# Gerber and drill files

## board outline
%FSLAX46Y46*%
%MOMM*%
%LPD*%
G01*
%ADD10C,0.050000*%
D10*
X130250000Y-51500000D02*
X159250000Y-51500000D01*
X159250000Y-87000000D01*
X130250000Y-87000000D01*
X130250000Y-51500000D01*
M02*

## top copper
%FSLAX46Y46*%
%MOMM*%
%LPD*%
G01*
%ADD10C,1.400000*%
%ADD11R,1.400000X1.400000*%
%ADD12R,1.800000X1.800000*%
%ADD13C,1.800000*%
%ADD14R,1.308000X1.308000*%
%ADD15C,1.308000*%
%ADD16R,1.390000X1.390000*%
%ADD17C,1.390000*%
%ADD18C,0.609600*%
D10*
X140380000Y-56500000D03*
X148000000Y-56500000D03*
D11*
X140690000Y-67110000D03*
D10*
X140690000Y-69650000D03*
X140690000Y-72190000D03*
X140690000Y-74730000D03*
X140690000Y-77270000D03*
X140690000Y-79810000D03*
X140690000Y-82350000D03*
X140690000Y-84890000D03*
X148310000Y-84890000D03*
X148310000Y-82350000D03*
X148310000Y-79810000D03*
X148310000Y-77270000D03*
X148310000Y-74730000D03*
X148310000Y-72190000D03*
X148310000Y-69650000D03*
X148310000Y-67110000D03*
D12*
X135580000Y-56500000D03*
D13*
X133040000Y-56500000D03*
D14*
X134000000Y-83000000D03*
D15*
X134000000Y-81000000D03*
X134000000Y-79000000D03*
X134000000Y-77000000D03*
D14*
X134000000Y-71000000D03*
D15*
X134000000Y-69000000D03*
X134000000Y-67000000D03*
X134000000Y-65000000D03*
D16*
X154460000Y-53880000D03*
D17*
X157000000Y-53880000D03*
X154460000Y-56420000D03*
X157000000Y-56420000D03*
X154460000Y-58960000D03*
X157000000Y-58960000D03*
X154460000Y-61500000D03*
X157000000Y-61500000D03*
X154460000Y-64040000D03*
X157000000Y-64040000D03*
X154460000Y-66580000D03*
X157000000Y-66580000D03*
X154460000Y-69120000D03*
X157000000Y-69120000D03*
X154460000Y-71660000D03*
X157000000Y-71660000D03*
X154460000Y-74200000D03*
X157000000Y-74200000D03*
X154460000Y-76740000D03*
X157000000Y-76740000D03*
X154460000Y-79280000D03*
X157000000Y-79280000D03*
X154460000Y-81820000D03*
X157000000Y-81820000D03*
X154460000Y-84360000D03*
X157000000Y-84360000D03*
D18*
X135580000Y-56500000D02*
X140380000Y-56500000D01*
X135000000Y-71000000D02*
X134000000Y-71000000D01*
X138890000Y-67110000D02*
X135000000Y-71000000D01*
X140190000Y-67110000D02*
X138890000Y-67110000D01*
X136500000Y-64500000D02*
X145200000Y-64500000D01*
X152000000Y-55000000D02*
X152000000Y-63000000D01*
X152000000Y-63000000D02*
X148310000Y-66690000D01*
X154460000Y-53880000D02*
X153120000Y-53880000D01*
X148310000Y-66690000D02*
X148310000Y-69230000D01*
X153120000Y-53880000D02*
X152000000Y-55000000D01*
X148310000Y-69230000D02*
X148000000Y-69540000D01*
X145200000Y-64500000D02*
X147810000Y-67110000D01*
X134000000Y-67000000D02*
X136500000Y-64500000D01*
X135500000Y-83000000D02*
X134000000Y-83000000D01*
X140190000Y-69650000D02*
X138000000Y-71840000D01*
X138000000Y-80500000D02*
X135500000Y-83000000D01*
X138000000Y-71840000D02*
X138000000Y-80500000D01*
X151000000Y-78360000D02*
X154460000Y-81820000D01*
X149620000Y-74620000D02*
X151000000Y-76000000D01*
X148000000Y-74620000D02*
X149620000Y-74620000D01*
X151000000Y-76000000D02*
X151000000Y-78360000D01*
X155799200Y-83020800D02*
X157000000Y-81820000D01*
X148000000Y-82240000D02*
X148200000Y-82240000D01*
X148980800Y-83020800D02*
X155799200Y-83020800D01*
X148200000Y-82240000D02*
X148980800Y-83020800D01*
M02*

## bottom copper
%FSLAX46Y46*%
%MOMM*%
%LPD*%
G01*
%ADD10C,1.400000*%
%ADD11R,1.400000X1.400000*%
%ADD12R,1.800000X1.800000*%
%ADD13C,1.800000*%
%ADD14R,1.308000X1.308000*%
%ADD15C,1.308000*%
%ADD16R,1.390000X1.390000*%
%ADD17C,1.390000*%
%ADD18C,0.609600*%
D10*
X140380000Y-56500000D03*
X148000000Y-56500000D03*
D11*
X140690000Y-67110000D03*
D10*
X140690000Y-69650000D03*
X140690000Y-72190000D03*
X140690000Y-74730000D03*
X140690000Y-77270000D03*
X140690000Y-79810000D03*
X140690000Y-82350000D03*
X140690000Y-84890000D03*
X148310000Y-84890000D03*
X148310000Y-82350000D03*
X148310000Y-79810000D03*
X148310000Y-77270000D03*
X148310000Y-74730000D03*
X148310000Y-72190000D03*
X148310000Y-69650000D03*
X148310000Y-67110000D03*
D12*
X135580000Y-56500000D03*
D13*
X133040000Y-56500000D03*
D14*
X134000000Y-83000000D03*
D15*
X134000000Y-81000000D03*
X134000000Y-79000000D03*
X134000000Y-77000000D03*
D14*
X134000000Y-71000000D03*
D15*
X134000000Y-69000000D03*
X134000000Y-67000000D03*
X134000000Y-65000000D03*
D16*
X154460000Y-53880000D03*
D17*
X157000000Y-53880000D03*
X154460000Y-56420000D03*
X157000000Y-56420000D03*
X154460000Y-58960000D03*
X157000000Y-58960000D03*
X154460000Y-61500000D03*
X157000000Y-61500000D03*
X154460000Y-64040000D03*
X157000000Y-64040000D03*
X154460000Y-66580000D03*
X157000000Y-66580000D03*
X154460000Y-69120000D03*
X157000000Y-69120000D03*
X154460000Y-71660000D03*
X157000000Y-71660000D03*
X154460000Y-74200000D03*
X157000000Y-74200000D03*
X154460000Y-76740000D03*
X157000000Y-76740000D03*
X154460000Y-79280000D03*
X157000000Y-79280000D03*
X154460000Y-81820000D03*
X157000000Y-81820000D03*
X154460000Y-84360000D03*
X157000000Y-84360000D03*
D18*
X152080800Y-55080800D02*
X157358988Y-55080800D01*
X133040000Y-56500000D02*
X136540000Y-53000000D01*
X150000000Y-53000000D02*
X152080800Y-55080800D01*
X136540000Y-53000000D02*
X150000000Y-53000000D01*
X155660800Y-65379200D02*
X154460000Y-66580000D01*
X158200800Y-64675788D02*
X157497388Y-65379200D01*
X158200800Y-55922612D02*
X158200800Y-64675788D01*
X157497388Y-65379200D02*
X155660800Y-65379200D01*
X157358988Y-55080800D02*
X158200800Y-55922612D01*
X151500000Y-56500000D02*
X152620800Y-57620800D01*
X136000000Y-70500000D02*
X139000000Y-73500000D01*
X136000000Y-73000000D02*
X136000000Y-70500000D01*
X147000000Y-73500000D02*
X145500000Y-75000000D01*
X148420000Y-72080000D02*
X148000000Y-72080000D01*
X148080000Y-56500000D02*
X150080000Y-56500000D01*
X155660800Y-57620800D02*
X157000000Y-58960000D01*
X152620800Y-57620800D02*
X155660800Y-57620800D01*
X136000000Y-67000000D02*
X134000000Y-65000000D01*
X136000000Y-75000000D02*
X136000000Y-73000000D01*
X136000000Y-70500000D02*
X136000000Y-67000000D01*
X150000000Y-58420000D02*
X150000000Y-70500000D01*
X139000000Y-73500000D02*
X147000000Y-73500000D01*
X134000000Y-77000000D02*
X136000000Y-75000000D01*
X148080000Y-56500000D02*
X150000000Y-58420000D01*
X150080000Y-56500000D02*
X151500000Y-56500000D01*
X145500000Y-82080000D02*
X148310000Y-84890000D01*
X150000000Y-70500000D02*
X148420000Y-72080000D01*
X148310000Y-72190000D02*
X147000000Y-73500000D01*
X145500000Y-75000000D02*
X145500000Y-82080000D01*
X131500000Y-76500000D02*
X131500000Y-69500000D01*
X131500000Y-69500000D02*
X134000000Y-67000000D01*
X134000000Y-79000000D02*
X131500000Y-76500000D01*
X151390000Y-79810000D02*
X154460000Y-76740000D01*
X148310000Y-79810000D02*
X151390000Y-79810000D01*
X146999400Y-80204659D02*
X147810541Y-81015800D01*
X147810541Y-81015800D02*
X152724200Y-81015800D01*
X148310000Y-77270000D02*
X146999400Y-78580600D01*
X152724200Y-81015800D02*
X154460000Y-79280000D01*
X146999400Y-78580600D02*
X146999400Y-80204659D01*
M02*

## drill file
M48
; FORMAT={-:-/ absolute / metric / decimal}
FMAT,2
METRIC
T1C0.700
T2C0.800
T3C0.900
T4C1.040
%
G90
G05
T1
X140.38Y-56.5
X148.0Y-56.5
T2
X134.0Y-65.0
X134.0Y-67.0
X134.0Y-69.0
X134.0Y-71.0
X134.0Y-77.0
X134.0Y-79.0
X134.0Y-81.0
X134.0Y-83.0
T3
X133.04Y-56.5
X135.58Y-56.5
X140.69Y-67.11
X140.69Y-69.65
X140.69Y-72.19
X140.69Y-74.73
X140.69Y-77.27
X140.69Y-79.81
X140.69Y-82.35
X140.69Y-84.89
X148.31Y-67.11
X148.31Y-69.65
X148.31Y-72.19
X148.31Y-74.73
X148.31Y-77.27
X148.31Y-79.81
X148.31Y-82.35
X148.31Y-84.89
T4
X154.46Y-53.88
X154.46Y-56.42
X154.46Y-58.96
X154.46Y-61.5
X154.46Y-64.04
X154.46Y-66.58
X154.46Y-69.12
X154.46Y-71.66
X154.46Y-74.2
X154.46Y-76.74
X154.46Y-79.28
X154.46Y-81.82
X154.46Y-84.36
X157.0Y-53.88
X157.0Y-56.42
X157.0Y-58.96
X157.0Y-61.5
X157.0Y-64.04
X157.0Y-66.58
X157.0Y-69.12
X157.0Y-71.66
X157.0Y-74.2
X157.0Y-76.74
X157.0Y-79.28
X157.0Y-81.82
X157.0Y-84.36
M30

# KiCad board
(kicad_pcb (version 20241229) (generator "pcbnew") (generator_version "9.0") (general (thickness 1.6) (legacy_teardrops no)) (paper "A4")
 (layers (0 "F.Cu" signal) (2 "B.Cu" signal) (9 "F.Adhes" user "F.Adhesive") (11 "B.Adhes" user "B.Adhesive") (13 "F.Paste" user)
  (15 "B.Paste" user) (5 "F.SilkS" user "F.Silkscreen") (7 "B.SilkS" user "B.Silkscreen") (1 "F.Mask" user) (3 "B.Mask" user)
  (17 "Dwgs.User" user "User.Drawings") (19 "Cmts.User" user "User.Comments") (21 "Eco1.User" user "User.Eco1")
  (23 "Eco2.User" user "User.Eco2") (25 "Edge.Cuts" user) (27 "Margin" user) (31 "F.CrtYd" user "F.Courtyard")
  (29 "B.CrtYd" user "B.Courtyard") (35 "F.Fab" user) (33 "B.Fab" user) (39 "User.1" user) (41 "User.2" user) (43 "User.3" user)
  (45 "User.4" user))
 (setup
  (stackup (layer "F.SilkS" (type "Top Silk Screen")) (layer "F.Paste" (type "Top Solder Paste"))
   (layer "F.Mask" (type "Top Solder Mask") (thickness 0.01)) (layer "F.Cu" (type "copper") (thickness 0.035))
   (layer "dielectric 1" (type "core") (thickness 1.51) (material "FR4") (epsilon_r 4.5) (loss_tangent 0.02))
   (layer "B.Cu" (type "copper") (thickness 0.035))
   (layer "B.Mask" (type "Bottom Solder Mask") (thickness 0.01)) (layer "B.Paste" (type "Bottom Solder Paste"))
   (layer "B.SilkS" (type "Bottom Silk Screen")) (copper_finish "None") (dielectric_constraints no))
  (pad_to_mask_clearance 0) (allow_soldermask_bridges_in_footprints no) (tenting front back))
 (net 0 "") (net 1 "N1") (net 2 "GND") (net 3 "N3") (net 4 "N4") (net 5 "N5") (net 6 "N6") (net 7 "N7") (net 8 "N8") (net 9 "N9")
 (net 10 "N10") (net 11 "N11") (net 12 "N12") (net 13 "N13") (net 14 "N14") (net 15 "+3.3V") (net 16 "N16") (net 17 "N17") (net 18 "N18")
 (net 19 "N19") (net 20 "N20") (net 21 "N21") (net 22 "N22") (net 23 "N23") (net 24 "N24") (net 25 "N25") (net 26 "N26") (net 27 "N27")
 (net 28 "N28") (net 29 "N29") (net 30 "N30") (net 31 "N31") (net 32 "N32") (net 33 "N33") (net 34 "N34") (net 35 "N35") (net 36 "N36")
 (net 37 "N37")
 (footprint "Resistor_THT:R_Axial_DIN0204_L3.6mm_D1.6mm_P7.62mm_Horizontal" (layer "F.Cu") (at 140.38 56.5)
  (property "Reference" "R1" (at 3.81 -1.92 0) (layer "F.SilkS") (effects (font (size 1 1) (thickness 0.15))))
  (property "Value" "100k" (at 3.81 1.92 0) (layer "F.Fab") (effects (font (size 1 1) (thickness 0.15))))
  (pad "1" thru_hole circle (at 0 0) (size 1.4 1.4) (drill 0.7) (layers "*.Cu" "*.Mask") (remove_unused_layers no) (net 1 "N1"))
  (pad "2" thru_hole circle (at 7.62 0) (size 1.4 1.4) (drill 0.7) (layers "*.Cu" "*.Mask") (remove_unused_layers no) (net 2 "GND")))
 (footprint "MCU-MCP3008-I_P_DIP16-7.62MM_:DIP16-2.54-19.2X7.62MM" (layer "F.Cu") (at 144.5 76 -90)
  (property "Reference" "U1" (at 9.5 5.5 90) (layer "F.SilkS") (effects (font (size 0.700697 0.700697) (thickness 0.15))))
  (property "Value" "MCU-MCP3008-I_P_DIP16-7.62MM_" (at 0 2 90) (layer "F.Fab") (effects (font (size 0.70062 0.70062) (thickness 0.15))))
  (pad "1" thru_hole rect (at -8.89 3.81 270) (size 1.4 1.4) (drill 0.9) (layers "*.Cu" "*.Mask") (remove_unused_layers no) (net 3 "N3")
   (solder_mask_margin 0.102))
  (pad "2" thru_hole circle (at -6.35 3.81 270) (size 1.4 1.4) (drill 0.9) (layers "*.Cu" "*.Mask") (remove_unused_layers no) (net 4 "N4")
   (solder_mask_margin 0.102))
  (pad "3" thru_hole circle (at -3.81 3.81 270) (size 1.4 1.4) (drill 0.9) (layers "*.Cu" "*.Mask") (remove_unused_layers no) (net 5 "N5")
   (solder_mask_margin 0.102))
  (pad "4" thru_hole circle (at -1.27 3.81 270) (size 1.4 1.4) (drill 0.9) (layers "*.Cu" "*.Mask") (remove_unused_layers no) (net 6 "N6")
   (solder_mask_margin 0.102))
  (pad "5" thru_hole circle (at 1.27 3.81 270) (size 1.4 1.4) (drill 0.9) (layers "*.Cu" "*.Mask") (remove_unused_layers no) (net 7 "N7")
   (solder_mask_margin 0.102))
  (pad "6" thru_hole circle (at 3.81 3.81 270) (size 1.4 1.4) (drill 0.9) (layers "*.Cu" "*.Mask") (remove_unused_layers no) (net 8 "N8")
   (solder_mask_margin 0.102))
  (pad "7" thru_hole circle (at 6.35 3.81 270) (size 1.4 1.4) (drill 0.9) (layers "*.Cu" "*.Mask") (remove_unused_layers no) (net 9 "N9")
   (solder_mask_margin 0.102))
  (pad "8" thru_hole circle (at 8.89 3.81 270) (size 1.4 1.4) (drill 0.9) (layers "*.Cu" "*.Mask") (remove_unused_layers no) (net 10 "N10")
   (solder_mask_margin 0.102))
  (pad "9" thru_hole circle (at 8.89 -3.81 270) (size 1.4 1.4) (drill 0.9) (layers "*.Cu" "*.Mask") (remove_unused_layers no) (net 2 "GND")
   (solder_mask_margin 0.102))
  (pad "10" thru_hole circle (at 6.35 -3.81 270) (size 1.4 1.4) (drill 0.9) (layers "*.Cu" "*.Mask") (remove_unused_layers no)
   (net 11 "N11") (solder_mask_margin 0.102))
  (pad "11" thru_hole circle (at 3.81 -3.81 270) (size 1.4 1.4) (drill 0.9) (layers "*.Cu" "*.Mask") (remove_unused_layers no)
   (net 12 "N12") (solder_mask_margin 0.102))
  (pad "12" thru_hole circle (at 1.27 -3.81 270) (size 1.4 1.4) (drill 0.9) (layers "*.Cu" "*.Mask") (remove_unused_layers no)
   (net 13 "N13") (solder_mask_margin 0.102))
  (pad "13" thru_hole circle (at -1.27 -3.81 270) (size 1.4 1.4) (drill 0.9) (layers "*.Cu" "*.Mask") (remove_unused_layers no)
   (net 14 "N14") (solder_mask_margin 0.102))
  (pad "14" thru_hole circle (at -3.81 -3.81 270) (size 1.4 1.4) (drill 0.9) (layers "*.Cu" "*.Mask") (remove_unused_layers no)
   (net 2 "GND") (solder_mask_margin 0.102))
  (pad "15" thru_hole circle (at -6.35 -3.81 270) (size 1.4 1.4) (drill 0.9) (layers "*.Cu" "*.Mask") (remove_unused_layers no)
   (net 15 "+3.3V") (solder_mask_margin 0.102))
  (pad "16" thru_hole circle (at -8.89 -3.81 270) (size 1.4 1.4) (drill 0.9) (layers "*.Cu" "*.Mask") (remove_unused_layers no)
   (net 15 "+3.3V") (solder_mask_margin 0.102)))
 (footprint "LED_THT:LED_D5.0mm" (layer "F.Cu") (at 135.58 56.5 180)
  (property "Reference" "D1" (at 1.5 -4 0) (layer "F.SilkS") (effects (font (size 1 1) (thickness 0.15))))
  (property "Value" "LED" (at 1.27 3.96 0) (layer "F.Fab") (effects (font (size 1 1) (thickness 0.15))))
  (pad "1" thru_hole rect (at 0 0 180) (size 1.8 1.8) (drill 0.9) (layers "*.Cu" "*.Mask") (remove_unused_layers no) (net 1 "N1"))
  (pad "2" thru_hole circle (at 2.54 0 180) (size 1.8 1.8) (drill 0.9) (layers "*.Cu" "*.Mask") (remove_unused_layers no) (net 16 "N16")))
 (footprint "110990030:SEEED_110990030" (layer "F.Cu") (at 134 80 90)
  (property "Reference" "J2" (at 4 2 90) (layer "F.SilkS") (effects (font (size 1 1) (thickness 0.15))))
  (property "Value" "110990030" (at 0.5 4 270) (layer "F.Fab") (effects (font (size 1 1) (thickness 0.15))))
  (pad "1" thru_hole rect (at -3 0 90) (size 1.308 1.308) (drill 0.8) (layers "*.Cu" "*.Mask") (remove_unused_layers no) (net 4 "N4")
   (solder_mask_margin 0.102))
  (pad "2" thru_hole circle (at -1 0 90) (size 1.308 1.308) (drill 0.8) (layers "*.Cu" "*.Mask") (remove_unused_layers no) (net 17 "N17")
   (solder_mask_margin 0.102))
  (pad "3" thru_hole circle (at 1 0 90) (size 1.308 1.308) (drill 0.8) (layers "*.Cu" "*.Mask") (remove_unused_layers no) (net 15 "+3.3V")
   (solder_mask_margin 0.102))
  (pad "4" thru_hole circle (at 3 0 90) (size 1.308 1.308) (drill 0.8) (layers "*.Cu" "*.Mask") (remove_unused_layers no) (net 2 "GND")
   (solder_mask_margin 0.102)))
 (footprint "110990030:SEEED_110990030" (layer "F.Cu") (at 134 68 90)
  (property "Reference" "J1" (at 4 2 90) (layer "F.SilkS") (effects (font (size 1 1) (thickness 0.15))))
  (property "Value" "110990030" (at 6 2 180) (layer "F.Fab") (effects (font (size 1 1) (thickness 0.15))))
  (pad "1" thru_hole rect (at -3 0 90) (size 1.308 1.308) (drill 0.8) (layers "*.Cu" "*.Mask") (remove_unused_layers no) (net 3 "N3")
   (solder_mask_margin 0.102))
  (pad "2" thru_hole circle (at -1 0 90) (size 1.308 1.308) (drill 0.8) (layers "*.Cu" "*.Mask") (remove_unused_layers no) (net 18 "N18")
   (solder_mask_margin 0.102))
  (pad "3" thru_hole circle (at 1 0 90) (size 1.308 1.308) (drill 0.8) (layers "*.Cu" "*.Mask") (remove_unused_layers no) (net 15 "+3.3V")
   (solder_mask_margin 0.102))
  (pad "4" thru_hole circle (at 3 0 90) (size 1.308 1.308) (drill 0.8) (layers "*.Cu" "*.Mask") (remove_unused_layers no) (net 2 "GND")
   (solder_mask_margin 0.102)))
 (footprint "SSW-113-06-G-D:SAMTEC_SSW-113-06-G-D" (layer "B.Cu") (at 154.46 53.88 90)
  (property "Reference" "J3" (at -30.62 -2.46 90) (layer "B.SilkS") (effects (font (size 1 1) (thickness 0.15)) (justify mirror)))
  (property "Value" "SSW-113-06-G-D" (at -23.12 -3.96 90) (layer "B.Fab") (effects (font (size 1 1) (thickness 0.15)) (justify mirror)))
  (pad "01" thru_hole rect (at 0 0 90) (size 1.39 1.39) (drill 1.04) (layers "*.Cu" "*.Mask") (remove_unused_layers no) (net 15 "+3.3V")
   (solder_mask_margin 0.102))
  (pad "02" thru_hole circle (at 0 2.54 90) (size 1.39 1.39) (drill 1.04) (layers "*.Cu" "*.Mask") (remove_unused_layers no) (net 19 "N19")
   (solder_mask_margin 0.102))
  (pad "03" thru_hole circle (at -2.54 0 90) (size 1.39 1.39) (drill 1.04) (layers "*.Cu" "*.Mask") (remove_unused_layers no) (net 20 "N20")
   (solder_mask_margin 0.102))
  (pad "04" thru_hole circle (at -2.54 2.54 90) (size 1.39 1.39) (drill 1.04) (layers "*.Cu" "*.Mask") (remove_unused_layers no)
   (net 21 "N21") (solder_mask_margin 0.102))
  (pad "05" thru_hole circle (at -5.08 0 90) (size 1.39 1.39) (drill 1.04) (layers "*.Cu" "*.Mask") (remove_unused_layers no) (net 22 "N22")
   (solder_mask_margin 0.102))
  (pad "06" thru_hole circle (at -5.08 2.54 90) (size 1.39 1.39) (drill 1.04) (layers "*.Cu" "*.Mask") (remove_unused_layers no)
   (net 2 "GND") (solder_mask_margin 0.102))
  (pad "07" thru_hole circle (at -7.62 0 90) (size 1.39 1.39) (drill 1.04) (layers "*.Cu" "*.Mask") (remove_unused_layers no) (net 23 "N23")
   (solder_mask_margin 0.102))
  (pad "08" thru_hole circle (at -7.62 2.54 90) (size 1.39 1.39) (drill 1.04) (layers "*.Cu" "*.Mask") (remove_unused_layers no)
   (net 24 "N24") (solder_mask_margin 0.102))
  (pad "09" thru_hole circle (at -10.16 0 90) (size 1.39 1.39) (drill 1.04) (layers "*.Cu" "*.Mask") (remove_unused_layers no)
   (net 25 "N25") (solder_mask_margin 0.102))
  (pad "10" thru_hole circle (at -10.16 2.54 90) (size 1.39 1.39) (drill 1.04) (layers "*.Cu" "*.Mask") (remove_unused_layers no)
   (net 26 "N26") (solder_mask_margin 0.102))
  (pad "11" thru_hole circle (at -12.7 0 90) (size 1.39 1.39) (drill 1.04) (layers "*.Cu" "*.Mask") (remove_unused_layers no) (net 16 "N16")
   (solder_mask_margin 0.102))
  (pad "12" thru_hole circle (at -12.7 2.54 90) (size 1.39 1.39) (drill 1.04) (layers "*.Cu" "*.Mask") (remove_unused_layers no)
   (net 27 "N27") (solder_mask_margin 0.102))
  (pad "13" thru_hole circle (at -15.24 0 90) (size 1.39 1.39) (drill 1.04) (layers "*.Cu" "*.Mask") (remove_unused_layers no)
   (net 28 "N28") (solder_mask_margin 0.102))
  (pad "14" thru_hole circle (at -15.24 2.54 90) (size 1.39 1.39) (drill 1.04) (layers "*.Cu" "*.Mask") (remove_unused_layers no)
   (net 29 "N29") (solder_mask_margin 0.102))
  (pad "15" thru_hole circle (at -17.78 0 90) (size 1.39 1.39) (drill 1.04) (layers "*.Cu" "*.Mask") (remove_unused_layers no)
   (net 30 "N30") (solder_mask_margin 0.102))
  (pad "16" thru_hole circle (at -17.78 2.54 90) (size 1.39 1.39) (drill 1.04) (layers "*.Cu" "*.Mask") (remove_unused_layers no)
   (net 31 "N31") (solder_mask_margin 0.102))
  (pad "17" thru_hole circle (at -20.32 0 90) (size 1.39 1.39) (drill 1.04) (layers "*.Cu" "*.Mask") (remove_unused_layers no)
   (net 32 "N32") (solder_mask_margin 0.102))
  (pad "18" thru_hole circle (at -20.32 2.54 90) (size 1.39 1.39) (drill 1.04) (layers "*.Cu" "*.Mask") (remove_unused_layers no)
   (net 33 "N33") (solder_mask_margin 0.102))
  (pad "19" thru_hole circle (at -22.86 0 90) (size 1.39 1.39) (drill 1.04) (layers "*.Cu" "*.Mask") (remove_unused_layers no)
   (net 12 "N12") (solder_mask_margin 0.102))
  (pad "20" thru_hole circle (at -22.86 2.54 90) (size 1.39 1.39) (drill 1.04) (layers "*.Cu" "*.Mask") (remove_unused_layers no)
   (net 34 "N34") (solder_mask_margin 0.102))
  (pad "21" thru_hole circle (at -25.4 0 90) (size 1.39 1.39) (drill 1.04) (layers "*.Cu" "*.Mask") (remove_unused_layers no) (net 13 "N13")
   (solder_mask_margin 0.102))
  (pad "22" thru_hole circle (at -25.4 2.54 90) (size 1.39 1.39) (drill 1.04) (layers "*.Cu" "*.Mask") (remove_unused_layers no)
   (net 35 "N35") (solder_mask_margin 0.102))
  (pad "23" thru_hole circle (at -27.94 0 90) (size 1.39 1.39) (drill 1.04) (layers "*.Cu" "*.Mask") (remove_unused_layers no)
   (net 14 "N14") (solder_mask_margin 0.102))
  (pad "24" thru_hole circle (at -27.94 2.54 90) (size 1.39 1.39) (drill 1.04) (layers "*.Cu" "*.Mask") (remove_unused_layers no)
   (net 11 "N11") (solder_mask_margin 0.102))
  (pad "25" thru_hole circle (at -30.48 0 90) (size 1.39 1.39) (drill 1.04) (layers "*.Cu" "*.Mask") (remove_unused_layers no)
   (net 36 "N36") (solder_mask_margin 0.102))
  (pad "26" thru_hole circle (at -30.48 2.54 90) (size 1.39 1.39) (drill 1.04) (layers "*.Cu" "*.Mask") (remove_unused_layers no)
   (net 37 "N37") (solder_mask_margin 0.102)))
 (gr_rect (start 130.25 51.5) (end 159.25 87) (stroke (width 0.05) (type default)) (fill no) (layer "Edge.Cuts"))
 (segment (start 135.58 56.5) (end 140.38 56.5) (width 0.6096) (layer "F.Cu") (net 1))
 (segment (start 152.0808 55.0808) (end 157.358988 55.0808) (width 0.6096) (layer "B.Cu") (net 16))
 (segment (start 133.04 56.5) (end 136.54 53) (width 0.6096) (layer "B.Cu") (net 16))
 (segment (start 150 53) (end 152.0808 55.0808) (width 0.6096) (layer "B.Cu") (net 16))
 (segment (start 136.54 53) (end 150 53) (width 0.6096) (layer "B.Cu") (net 16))
 (segment (start 155.6608 65.3792) (end 154.46 66.58) (width 0.6096) (layer "B.Cu") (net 16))
 (segment (start 158.2008 64.675788) (end 157.497388 65.3792) (width 0.6096) (layer "B.Cu") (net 16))
 (segment (start 158.2008 55.922612) (end 158.2008 64.675788) (width 0.6096) (layer "B.Cu") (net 16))
 (segment (start 157.497388 65.3792) (end 155.6608 65.3792) (width 0.6096) (layer "B.Cu") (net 16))
 (segment (start 157.358988 55.0808) (end 158.2008 55.922612) (width 0.6096) (layer "B.Cu") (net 16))
 (segment (start 135 71) (end 134 71) (width 0.6096) (layer "F.Cu") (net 3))
 (segment (start 138.89 67.11) (end 135 71) (width 0.6096) (layer "F.Cu") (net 3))
 (segment (start 140.19 67.11) (end 138.89 67.11) (width 0.6096) (layer "F.Cu") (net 3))
 (segment (start 151.5 56.5) (end 152.6208 57.6208) (width 0.6096) (layer "B.Cu") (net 2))
 (segment (start 136 70.5) (end 139 73.5) (width 0.6096) (layer "B.Cu") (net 2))
 (segment (start 136 73) (end 136 70.5) (width 0.6096) (layer "B.Cu") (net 2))
 (segment (start 147 73.5) (end 145.5 75) (width 0.6096) (layer "B.Cu") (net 2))
 (segment (start 148.42 72.08) (end 148 72.08) (width 0.6096) (layer "B.Cu") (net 2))
 (segment (start 148.08 56.5) (end 150.08 56.5) (width 0.6096) (layer "B.Cu") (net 2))
 (segment (start 155.6608 57.6208) (end 157 58.96) (width 0.6096) (layer "B.Cu") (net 2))
 (segment (start 152.6208 57.6208) (end 155.6608 57.6208) (width 0.6096) (layer "B.Cu") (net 2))
 (segment (start 136 67) (end 134 65) (width 0.6096) (layer "B.Cu") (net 2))
 (segment (start 136 75) (end 136 73) (width 0.6096) (layer "B.Cu") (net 2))
 (segment (start 136 70.5) (end 136 67) (width 0.6096) (layer "B.Cu") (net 2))
 (segment (start 150 58.42) (end 150 70.5) (width 0.6096) (layer "B.Cu") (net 2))
 (segment (start 139 73.5) (end 147 73.5) (width 0.6096) (layer "B.Cu") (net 2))
 (segment (start 134 77) (end 136 75) (width 0.6096) (layer "B.Cu") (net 2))
 (segment (start 148.08 56.5) (end 150 58.42) (width 0.6096) (layer "B.Cu") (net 2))
 (segment (start 150.08 56.5) (end 151.5 56.5) (width 0.6096) (layer "B.Cu") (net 2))
 (segment (start 145.5 82.08) (end 148.31 84.89) (width 0.6096) (layer "B.Cu") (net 2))
 (segment (start 150 70.5) (end 148.42 72.08) (width 0.6096) (layer "B.Cu") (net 2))
 (segment (start 148.31 72.19) (end 147 73.5) (width 0.6096) (layer "B.Cu") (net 2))
 (segment (start 145.5 75) (end 145.5 82.08) (width 0.6096) (layer "B.Cu") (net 2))
 (segment (start 136.5 64.5) (end 145.2 64.5) (width 0.6096) (layer "F.Cu") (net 15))
 (segment (start 152 55) (end 152 63) (width 0.6096) (layer "F.Cu") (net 15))
 (segment (start 152 63) (end 148.31 66.69) (width 0.6096) (layer "F.Cu") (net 15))
 (segment (start 154.46 53.88) (end 153.12 53.88) (width 0.6096) (layer "F.Cu") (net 15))
 (segment (start 148.31 66.69) (end 148.31 69.23) (width 0.6096) (layer "F.Cu") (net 15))
 (segment (start 153.12 53.88) (end 152 55) (width 0.6096) (layer "F.Cu") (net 15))
 (segment (start 148.31 69.23) (end 148 69.54) (width 0.6096) (layer "F.Cu") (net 15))
 (segment (start 145.2 64.5) (end 147.81 67.11) (width 0.6096) (layer "F.Cu") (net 15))
 (segment (start 134 67) (end 136.5 64.5) (width 0.6096) (layer "F.Cu") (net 15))
 (segment (start 131.5 76.5) (end 131.5 69.5) (width 0.6096) (layer "B.Cu") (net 15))
 (segment (start 131.5 69.5) (end 134 67) (width 0.6096) (layer "B.Cu") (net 15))
 (segment (start 134 79) (end 131.5 76.5) (width 0.6096) (layer "B.Cu") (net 15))
 (segment (start 135.5 83) (end 134 83) (width 0.6096) (layer "F.Cu") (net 4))
 (segment (start 140.19 69.65) (end 138 71.84) (width 0.6096) (layer "F.Cu") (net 4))
 (segment (start 138 80.5) (end 135.5 83) (width 0.6096) (layer "F.Cu") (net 4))
 (segment (start 138 71.84) (end 138 80.5) (width 0.6096) (layer "F.Cu") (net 4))
 (segment (start 151.39 79.81) (end 154.46 76.74) (width 0.6096) (layer "B.Cu") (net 12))
 (segment (start 148.31 79.81) (end 151.39 79.81) (width 0.6096) (layer "B.Cu") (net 12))
 (segment (start 151 78.36) (end 154.46 81.82) (width 0.6096) (layer "F.Cu") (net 14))
 (segment (start 149.62 74.62) (end 151 76) (width 0.6096) (layer "F.Cu") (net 14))
 (segment (start 148 74.62) (end 149.62 74.62) (width 0.6096) (layer "F.Cu") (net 14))
 (segment (start 151 76) (end 151 78.36) (width 0.6096) (layer "F.Cu") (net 14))
 (segment (start 155.7992 83.0208) (end 157 81.82) (width 0.6096) (layer "F.Cu") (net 11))
 (segment (start 148 82.24) (end 148.2 82.24) (width 0.6096) (layer "F.Cu") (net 11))
 (segment (start 148.9808 83.0208) (end 155.7992 83.0208) (width 0.6096) (layer "F.Cu") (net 11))
 (segment (start 148.2 82.24) (end 148.9808 83.0208) (width 0.6096) (layer "F.Cu") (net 11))
 (segment (start 146.9994 80.204659) (end 147.810541 81.0158) (width 0.6096) (layer "B.Cu") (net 13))
 (segment (start 147.810541 81.0158) (end 152.7242 81.0158) (width 0.6096) (layer "B.Cu") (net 13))
 (segment (start 148.31 77.27) (end 146.9994 78.5806) (width 0.6096) (layer "B.Cu") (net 13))
 (segment (start 152.7242 81.0158) (end 154.46 79.28) (width 0.6096) (layer "B.Cu") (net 13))
 (segment (start 146.9994 78.5806) (end 146.9994 80.204659) (width 0.6096) (layer "B.Cu") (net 13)))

